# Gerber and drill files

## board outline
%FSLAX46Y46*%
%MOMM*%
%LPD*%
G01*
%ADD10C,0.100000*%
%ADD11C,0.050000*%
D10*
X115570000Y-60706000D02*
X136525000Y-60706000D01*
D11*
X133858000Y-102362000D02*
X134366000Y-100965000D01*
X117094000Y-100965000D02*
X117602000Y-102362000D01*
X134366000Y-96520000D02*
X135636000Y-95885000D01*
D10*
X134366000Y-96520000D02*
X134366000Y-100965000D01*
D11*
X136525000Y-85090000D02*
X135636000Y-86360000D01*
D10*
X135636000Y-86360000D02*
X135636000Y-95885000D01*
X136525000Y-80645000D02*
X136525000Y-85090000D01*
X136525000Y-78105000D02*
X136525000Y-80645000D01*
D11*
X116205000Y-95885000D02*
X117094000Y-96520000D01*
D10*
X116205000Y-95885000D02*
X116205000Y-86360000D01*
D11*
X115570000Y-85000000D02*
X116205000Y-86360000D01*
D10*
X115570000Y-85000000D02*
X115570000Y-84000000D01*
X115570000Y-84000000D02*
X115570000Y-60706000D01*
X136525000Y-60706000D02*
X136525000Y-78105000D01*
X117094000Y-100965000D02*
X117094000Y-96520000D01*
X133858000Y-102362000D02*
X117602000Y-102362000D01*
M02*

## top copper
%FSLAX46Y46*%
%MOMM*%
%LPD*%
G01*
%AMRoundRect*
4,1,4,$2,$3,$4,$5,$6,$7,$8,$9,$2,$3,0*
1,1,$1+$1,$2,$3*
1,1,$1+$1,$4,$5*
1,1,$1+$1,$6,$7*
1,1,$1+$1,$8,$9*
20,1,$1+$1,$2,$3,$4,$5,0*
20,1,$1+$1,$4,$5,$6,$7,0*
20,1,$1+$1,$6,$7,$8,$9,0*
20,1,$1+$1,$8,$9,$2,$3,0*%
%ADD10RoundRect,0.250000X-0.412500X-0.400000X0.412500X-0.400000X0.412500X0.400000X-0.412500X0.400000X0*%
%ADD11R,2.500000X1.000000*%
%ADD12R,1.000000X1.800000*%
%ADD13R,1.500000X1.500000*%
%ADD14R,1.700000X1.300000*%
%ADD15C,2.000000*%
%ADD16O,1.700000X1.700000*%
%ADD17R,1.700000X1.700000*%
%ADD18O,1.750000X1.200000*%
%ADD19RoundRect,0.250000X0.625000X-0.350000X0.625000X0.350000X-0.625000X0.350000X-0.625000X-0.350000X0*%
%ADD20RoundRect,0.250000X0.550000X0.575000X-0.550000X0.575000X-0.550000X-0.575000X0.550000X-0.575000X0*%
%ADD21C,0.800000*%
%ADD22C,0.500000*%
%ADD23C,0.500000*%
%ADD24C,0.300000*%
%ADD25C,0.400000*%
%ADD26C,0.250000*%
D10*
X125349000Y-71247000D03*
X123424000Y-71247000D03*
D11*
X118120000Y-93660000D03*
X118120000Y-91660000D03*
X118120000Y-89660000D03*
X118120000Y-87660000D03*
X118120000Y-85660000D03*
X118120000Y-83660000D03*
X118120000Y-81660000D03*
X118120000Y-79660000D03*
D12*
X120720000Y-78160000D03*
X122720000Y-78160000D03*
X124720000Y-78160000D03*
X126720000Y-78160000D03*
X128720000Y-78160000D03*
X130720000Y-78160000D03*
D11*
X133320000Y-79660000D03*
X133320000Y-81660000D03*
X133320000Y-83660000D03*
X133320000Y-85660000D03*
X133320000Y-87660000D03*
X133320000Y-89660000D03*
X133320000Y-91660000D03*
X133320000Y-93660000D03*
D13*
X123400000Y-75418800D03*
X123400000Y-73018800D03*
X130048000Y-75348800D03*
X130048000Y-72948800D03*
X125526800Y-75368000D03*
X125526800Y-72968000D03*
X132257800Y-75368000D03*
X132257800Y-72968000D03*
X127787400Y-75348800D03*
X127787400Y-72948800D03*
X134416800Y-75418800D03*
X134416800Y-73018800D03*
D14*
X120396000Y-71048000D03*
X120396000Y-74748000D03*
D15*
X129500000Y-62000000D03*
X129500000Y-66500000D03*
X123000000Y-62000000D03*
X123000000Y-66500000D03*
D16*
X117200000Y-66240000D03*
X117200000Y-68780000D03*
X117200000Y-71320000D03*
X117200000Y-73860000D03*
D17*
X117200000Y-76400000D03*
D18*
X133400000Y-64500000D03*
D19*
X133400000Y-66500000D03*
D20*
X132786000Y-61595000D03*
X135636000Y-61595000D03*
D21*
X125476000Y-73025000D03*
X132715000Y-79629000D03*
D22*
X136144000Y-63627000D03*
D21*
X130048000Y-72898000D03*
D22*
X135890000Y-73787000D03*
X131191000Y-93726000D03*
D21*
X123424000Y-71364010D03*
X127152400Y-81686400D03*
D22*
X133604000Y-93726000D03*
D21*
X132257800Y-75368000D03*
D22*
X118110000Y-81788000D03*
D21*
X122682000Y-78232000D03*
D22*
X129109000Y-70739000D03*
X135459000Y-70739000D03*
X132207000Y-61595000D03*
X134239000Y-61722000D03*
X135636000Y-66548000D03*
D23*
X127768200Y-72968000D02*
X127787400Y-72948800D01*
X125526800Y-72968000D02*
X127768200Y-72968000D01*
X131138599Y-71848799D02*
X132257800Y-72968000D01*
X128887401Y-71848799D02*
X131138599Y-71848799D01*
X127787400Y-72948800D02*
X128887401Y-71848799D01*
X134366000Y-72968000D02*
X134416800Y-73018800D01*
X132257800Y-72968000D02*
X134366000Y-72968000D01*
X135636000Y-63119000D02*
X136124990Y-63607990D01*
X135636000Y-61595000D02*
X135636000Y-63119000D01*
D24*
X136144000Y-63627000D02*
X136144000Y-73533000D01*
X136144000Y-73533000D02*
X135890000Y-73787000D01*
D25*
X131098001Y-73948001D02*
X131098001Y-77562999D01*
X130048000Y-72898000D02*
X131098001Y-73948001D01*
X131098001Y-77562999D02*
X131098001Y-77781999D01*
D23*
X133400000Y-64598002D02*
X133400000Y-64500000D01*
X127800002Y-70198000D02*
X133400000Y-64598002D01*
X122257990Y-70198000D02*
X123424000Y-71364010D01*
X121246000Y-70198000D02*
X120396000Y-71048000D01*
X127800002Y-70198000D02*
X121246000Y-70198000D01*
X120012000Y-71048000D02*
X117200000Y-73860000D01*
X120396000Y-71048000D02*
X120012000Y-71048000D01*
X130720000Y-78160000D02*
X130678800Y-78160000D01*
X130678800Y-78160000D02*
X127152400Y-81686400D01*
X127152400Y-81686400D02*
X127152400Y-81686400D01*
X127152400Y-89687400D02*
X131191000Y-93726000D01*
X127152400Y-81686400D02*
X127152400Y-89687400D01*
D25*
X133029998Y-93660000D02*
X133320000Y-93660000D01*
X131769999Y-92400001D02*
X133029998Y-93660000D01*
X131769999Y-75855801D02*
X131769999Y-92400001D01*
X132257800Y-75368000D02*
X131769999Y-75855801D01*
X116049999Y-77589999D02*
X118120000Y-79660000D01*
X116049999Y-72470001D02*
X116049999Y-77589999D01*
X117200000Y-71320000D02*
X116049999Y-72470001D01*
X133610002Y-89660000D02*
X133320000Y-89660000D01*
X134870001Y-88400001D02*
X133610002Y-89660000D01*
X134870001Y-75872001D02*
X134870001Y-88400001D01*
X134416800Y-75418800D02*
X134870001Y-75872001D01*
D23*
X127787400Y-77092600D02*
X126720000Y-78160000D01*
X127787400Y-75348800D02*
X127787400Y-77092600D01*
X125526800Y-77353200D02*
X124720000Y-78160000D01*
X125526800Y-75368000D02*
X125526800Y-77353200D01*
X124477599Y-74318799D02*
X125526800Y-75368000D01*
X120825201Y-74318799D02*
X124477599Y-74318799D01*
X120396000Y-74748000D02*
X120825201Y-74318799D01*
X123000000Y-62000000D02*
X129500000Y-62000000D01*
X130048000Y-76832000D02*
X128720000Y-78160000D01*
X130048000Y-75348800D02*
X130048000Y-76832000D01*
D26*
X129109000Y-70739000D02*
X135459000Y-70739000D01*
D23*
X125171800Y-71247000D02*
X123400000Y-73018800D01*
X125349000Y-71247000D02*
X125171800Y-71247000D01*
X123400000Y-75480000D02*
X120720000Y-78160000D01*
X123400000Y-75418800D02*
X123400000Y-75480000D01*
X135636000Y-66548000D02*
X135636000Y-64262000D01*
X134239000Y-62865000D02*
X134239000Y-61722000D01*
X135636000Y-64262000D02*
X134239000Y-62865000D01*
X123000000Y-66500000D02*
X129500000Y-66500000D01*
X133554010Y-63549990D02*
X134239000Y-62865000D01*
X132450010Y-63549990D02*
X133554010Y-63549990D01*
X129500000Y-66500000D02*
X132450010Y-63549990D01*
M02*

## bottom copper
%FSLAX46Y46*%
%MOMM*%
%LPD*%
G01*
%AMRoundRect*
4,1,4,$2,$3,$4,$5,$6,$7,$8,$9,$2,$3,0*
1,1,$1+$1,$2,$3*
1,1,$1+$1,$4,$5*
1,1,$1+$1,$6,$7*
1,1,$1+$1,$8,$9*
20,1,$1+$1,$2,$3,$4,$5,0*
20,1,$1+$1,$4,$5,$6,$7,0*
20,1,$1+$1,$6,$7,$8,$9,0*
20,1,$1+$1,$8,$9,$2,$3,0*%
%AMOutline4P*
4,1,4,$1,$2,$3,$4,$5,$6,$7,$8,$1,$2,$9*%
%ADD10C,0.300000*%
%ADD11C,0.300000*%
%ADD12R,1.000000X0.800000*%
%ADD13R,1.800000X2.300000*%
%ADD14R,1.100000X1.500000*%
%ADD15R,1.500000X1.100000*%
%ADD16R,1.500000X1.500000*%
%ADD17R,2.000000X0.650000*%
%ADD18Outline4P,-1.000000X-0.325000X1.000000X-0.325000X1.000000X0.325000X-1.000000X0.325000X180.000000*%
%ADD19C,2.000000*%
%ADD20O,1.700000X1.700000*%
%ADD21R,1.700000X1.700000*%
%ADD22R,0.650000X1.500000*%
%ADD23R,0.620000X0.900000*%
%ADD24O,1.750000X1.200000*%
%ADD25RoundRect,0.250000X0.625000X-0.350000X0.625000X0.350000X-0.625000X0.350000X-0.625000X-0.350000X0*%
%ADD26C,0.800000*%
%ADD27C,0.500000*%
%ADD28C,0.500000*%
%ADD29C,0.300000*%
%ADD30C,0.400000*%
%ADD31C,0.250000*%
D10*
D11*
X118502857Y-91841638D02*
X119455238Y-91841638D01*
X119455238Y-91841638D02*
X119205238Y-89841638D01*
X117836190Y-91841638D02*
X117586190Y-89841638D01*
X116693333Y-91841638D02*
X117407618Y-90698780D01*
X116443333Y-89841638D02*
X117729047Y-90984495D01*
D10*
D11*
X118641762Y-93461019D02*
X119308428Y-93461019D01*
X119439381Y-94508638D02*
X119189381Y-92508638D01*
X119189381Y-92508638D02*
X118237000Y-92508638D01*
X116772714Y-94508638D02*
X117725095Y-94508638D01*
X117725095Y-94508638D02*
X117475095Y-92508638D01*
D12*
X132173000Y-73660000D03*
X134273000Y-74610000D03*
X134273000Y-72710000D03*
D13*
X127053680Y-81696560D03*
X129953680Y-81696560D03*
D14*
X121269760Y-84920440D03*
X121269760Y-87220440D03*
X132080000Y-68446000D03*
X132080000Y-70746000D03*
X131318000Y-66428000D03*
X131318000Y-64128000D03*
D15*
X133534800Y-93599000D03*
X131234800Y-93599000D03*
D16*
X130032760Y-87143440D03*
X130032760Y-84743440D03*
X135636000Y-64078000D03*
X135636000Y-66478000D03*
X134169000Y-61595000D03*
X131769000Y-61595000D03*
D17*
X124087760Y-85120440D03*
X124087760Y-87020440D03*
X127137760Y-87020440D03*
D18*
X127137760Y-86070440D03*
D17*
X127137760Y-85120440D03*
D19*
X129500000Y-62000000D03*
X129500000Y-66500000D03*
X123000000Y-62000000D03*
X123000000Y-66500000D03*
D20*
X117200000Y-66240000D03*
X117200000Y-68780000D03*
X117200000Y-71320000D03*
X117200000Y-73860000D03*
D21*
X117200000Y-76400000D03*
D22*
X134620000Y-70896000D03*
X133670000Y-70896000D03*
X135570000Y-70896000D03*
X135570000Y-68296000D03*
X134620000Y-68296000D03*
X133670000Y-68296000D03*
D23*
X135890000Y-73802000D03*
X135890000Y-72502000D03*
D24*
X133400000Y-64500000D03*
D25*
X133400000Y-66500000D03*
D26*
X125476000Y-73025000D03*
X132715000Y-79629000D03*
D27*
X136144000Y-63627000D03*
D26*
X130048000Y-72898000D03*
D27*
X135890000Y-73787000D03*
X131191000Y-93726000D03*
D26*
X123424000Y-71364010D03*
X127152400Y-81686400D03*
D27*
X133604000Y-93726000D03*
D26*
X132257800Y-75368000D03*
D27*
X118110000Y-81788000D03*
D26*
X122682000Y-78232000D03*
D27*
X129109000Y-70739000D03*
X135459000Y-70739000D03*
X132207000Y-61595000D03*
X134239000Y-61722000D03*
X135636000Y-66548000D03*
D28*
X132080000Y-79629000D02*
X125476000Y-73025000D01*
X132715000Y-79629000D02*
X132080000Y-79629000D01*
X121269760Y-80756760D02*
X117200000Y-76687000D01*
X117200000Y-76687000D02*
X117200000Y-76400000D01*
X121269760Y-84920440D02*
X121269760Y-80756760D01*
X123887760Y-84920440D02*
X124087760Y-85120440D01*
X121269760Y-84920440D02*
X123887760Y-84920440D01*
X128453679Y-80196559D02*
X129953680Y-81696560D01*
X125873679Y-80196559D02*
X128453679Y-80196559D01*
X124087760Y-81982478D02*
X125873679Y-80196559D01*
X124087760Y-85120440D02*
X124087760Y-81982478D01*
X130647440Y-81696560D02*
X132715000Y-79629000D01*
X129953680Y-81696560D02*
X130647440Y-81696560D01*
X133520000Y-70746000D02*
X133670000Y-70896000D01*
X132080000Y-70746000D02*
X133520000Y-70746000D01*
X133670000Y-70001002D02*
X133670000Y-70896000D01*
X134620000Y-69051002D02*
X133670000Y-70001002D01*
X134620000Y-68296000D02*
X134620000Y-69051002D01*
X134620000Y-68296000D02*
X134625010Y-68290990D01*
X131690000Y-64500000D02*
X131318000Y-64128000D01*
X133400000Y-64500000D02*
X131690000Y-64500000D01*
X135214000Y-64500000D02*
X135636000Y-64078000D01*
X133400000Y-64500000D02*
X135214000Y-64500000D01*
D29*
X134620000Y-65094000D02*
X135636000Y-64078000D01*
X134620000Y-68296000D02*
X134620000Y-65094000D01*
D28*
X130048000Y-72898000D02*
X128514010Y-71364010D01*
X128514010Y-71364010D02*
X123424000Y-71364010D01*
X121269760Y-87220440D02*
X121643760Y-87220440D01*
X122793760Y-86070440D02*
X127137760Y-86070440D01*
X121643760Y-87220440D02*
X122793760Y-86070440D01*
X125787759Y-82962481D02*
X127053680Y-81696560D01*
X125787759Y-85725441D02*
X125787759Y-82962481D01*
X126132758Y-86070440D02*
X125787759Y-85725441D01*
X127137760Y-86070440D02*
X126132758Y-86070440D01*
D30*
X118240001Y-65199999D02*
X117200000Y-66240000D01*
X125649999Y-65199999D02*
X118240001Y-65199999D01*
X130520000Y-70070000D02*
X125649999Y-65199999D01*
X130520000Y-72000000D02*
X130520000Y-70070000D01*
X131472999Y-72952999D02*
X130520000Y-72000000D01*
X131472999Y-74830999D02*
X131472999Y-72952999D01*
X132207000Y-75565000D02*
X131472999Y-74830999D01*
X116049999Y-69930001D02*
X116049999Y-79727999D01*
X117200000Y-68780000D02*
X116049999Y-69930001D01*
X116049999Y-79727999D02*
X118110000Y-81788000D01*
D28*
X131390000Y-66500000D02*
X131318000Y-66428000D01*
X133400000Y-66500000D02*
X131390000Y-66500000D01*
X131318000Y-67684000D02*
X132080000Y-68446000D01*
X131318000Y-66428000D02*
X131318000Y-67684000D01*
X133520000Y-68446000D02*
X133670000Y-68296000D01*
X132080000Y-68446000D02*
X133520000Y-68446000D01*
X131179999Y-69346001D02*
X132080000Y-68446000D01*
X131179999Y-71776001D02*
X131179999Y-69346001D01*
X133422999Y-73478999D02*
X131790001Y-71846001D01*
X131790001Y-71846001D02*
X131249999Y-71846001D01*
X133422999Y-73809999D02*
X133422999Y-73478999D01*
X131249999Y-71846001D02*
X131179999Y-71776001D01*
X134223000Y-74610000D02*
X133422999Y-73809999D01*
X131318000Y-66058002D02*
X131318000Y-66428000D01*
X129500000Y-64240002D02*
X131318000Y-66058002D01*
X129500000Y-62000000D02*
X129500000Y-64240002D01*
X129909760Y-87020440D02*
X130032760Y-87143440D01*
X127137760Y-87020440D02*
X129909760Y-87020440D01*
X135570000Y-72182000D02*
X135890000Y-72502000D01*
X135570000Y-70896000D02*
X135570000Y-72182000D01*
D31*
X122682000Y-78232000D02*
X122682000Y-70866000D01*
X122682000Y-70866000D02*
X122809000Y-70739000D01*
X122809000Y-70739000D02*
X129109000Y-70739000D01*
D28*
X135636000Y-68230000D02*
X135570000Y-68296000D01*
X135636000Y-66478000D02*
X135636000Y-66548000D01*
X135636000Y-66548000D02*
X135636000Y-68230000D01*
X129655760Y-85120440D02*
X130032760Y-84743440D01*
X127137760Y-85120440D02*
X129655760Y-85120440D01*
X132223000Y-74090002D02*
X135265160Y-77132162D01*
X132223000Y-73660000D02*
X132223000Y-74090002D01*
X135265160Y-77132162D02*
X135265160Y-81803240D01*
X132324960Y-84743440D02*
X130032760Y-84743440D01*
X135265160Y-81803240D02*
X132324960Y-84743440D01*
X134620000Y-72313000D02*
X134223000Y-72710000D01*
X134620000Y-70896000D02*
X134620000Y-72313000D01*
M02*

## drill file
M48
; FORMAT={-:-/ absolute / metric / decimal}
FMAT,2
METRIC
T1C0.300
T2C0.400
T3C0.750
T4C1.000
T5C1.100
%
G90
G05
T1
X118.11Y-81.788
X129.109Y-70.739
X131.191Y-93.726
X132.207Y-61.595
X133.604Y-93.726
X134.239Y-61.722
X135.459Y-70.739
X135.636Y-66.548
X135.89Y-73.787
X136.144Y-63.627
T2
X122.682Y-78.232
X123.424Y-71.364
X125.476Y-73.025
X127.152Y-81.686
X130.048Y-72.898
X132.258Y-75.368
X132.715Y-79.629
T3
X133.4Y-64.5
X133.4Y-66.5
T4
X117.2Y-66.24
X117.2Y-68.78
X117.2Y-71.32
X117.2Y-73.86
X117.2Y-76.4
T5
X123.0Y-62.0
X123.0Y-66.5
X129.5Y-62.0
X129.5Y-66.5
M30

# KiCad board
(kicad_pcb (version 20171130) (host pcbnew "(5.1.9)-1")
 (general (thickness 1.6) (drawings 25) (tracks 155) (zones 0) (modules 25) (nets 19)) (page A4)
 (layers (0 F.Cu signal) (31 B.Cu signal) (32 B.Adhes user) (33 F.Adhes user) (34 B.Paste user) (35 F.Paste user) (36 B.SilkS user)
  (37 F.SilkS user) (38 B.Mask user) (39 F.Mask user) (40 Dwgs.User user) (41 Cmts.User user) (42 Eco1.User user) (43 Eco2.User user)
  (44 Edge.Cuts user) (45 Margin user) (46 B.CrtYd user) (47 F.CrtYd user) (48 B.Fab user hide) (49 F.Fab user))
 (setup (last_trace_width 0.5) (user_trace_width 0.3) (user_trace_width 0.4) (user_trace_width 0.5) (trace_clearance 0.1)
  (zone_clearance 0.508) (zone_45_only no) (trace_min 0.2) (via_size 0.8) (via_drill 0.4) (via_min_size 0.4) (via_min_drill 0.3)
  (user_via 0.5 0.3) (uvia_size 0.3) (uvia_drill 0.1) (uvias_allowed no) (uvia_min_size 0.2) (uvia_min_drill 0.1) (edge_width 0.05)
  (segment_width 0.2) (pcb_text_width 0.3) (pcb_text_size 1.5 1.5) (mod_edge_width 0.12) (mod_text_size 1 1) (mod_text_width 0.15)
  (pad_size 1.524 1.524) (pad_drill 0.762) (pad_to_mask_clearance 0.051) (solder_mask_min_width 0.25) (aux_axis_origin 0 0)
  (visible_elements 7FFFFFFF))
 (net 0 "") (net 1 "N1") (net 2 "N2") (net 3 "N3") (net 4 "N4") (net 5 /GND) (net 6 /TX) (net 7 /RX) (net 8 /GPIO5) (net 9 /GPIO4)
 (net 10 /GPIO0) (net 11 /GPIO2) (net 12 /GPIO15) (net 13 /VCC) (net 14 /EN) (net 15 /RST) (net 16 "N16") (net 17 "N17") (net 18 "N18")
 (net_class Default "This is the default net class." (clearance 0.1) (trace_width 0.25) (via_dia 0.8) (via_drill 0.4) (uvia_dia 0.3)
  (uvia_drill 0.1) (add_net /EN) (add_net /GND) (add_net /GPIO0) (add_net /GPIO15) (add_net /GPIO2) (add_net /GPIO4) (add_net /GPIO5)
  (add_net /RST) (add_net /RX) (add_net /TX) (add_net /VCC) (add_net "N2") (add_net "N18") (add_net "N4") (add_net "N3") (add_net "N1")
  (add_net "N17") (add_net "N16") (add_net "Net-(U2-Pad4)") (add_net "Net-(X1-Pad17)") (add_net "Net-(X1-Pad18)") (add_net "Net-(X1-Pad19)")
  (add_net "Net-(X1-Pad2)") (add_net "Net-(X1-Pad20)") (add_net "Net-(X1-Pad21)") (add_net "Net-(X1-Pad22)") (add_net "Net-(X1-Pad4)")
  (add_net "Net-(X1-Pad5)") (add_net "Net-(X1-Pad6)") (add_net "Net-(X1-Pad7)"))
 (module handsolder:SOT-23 (layer B.Cu) (at 133.223 73.66 180)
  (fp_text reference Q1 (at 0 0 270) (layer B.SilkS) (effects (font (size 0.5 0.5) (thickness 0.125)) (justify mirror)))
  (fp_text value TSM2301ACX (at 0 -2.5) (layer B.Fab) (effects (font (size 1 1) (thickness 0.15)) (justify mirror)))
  (pad 3 smd rect (at 1.05 0 180) (size 1 0.8) (layers B.Cu B.Paste B.Mask) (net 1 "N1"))
  (pad 2 smd rect (at -1.05 -0.95 180) (size 1 0.8) (layers B.Cu B.Paste B.Mask) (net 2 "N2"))
  (pad 1 smd rect (at -1.05 0.95 180) (size 1 0.8) (layers B.Cu B.Paste B.Mask) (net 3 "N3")))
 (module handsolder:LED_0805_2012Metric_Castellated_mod (layer F.Cu) (at 124.3865 71.247)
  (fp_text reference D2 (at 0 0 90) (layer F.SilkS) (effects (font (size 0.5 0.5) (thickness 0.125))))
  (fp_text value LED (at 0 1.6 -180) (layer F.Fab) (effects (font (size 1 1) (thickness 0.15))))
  (pad 2 smd roundrect (at 0.9625 0) (size 1.325 1.3) (layers F.Cu F.Paste F.Mask) (roundrect_rratio 0.1923076923076923) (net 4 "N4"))
  (pad 1 smd roundrect (at -0.9625 0) (size 1.325 1.3) (layers F.Cu F.Paste F.Mask) (roundrect_rratio 0.1923076923076923) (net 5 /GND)))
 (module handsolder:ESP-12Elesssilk (layer F.Cu) (at 125.72 90.16 180)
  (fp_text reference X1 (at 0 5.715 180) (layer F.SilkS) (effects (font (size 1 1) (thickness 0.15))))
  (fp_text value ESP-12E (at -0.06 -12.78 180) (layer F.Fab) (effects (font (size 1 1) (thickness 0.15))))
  (pad 22 smd rect (at 7.6 -3.5 180) (size 2.5 1) (layers F.Cu F.Paste F.Mask))
  (pad 21 smd rect (at 7.6 -1.5 180) (size 2.5 1) (layers F.Cu F.Paste F.Mask))
  (pad 20 smd rect (at 7.6 0.5 180) (size 2.5 1) (layers F.Cu F.Paste F.Mask))
  (pad 19 smd rect (at 7.6 2.5 180) (size 2.5 1) (layers F.Cu F.Paste F.Mask))
  (pad 18 smd rect (at 7.6 4.5 180) (size 2.5 1) (layers F.Cu F.Paste F.Mask))
  (pad 17 smd rect (at 7.6 6.5 180) (size 2.5 1) (layers F.Cu F.Paste F.Mask))
  (pad 16 smd rect (at 7.6 8.5 180) (size 2.5 1) (layers F.Cu F.Paste F.Mask) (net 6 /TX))
  (pad 15 smd rect (at 7.6 10.5 180) (size 2.5 1) (layers F.Cu F.Paste F.Mask) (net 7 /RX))
  (pad 14 smd rect (at 5 12 180) (size 1 1.8) (layers F.Cu F.Paste F.Mask) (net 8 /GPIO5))
  (pad 13 smd rect (at 3 12 180) (size 1 1.8) (layers F.Cu F.Paste F.Mask) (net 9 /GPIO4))
  (pad 12 smd rect (at 1 12 180) (size 1 1.8) (layers F.Cu F.Paste F.Mask) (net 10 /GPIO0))
  (pad 11 smd rect (at -1 12 180) (size 1 1.8) (layers F.Cu F.Paste F.Mask) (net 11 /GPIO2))
  (pad 10 smd rect (at -3 12 180) (size 1 1.8) (layers F.Cu F.Paste F.Mask) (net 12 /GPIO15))
  (pad 9 smd rect (at -5 12 180) (size 1 1.8) (layers F.Cu F.Paste F.Mask) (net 5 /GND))
  (pad 8 smd rect (at -7.6 10.5 180) (size 2.5 1) (layers F.Cu F.Paste F.Mask) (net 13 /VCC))
  (pad 7 smd rect (at -7.6 8.5 180) (size 2.5 1) (layers F.Cu F.Paste F.Mask))
  (pad 6 smd rect (at -7.6 6.5 180) (size 2.5 1) (layers F.Cu F.Paste F.Mask))
  (pad 5 smd rect (at -7.6 4.5 180) (size 2.5 1) (layers F.Cu F.Paste F.Mask))
  (pad 4 smd rect (at -7.6 2.5 180) (size 2.5 1) (layers F.Cu F.Paste F.Mask))
  (pad 3 smd rect (at -7.6 0.5 180) (size 2.5 1) (layers F.Cu F.Paste F.Mask) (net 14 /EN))
  (pad 2 smd rect (at -7.6 -1.5 180) (size 2.5 1) (layers F.Cu F.Paste F.Mask))
  (pad 1 smd rect (at -7.6 -3.5 180) (size 2.5 1) (layers F.Cu F.Paste F.Mask) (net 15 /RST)))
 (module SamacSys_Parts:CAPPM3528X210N (layer B.Cu) (at 128.50368 81.69656 180)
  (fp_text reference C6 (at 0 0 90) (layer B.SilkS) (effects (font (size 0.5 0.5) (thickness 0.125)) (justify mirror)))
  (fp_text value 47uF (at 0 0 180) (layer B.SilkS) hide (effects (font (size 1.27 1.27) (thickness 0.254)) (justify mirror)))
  (pad 2 smd rect (at 1.45 0 180) (size 1.8 2.3) (layers B.Cu B.Paste B.Mask) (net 5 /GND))
  (pad 1 smd rect (at -1.45 0 180) (size 1.8 2.3) (layers B.Cu B.Paste B.Mask) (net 13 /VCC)))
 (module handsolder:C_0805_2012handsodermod (layer B.Cu) (at 121.26976 86.07044 90)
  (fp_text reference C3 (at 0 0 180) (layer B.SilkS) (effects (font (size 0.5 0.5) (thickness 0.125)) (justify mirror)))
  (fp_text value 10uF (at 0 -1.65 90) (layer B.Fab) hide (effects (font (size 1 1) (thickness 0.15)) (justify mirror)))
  (pad 2 smd rect (at 1.15 0 90) (size 1.5 1.1) (layers B.Cu B.Paste B.Mask) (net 13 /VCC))
  (pad 1 smd rect (at -1.15 0 90) (size 1.5 1.1) (layers B.Cu B.Paste B.Mask) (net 5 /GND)))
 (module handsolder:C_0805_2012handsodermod (layer B.Cu) (at 132.08 69.596 90)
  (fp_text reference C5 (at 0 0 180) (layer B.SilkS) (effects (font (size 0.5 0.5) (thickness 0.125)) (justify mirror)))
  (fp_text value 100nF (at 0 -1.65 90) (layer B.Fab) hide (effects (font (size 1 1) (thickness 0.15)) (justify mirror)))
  (pad 2 smd rect (at 1.15 0 90) (size 1.5 1.1) (layers B.Cu B.Paste B.Mask) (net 2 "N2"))
  (pad 1 smd rect (at -1.15 0 90) (size 1.5 1.1) (layers B.Cu B.Paste B.Mask) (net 5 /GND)))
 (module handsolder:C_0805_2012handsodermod (layer B.Cu) (at 131.318 65.278 270)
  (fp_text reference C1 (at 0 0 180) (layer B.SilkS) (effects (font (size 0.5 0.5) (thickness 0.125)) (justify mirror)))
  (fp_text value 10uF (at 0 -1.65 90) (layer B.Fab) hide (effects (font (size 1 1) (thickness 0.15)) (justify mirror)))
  (pad 2 smd rect (at 1.15 0 270) (size 1.5 1.1) (layers B.Cu B.Paste B.Mask) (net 2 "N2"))
  (pad 1 smd rect (at -1.15 0 270) (size 1.5 1.1) (layers B.Cu B.Paste B.Mask) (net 5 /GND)))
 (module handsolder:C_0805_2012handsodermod (layer B.Cu) (at 132.3848 93.599)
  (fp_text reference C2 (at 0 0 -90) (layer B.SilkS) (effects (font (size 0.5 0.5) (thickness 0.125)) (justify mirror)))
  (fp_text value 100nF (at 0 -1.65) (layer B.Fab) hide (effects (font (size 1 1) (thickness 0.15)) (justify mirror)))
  (pad 2 smd rect (at 1.15 0) (size 1.5 1.1) (layers B.Cu B.Paste B.Mask) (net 15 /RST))
  (pad 1 smd rect (at -1.15 0) (size 1.5 1.1) (layers B.Cu B.Paste B.Mask) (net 5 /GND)))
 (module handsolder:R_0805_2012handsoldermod (layer F.Cu) (at 123.4 74.2188 270)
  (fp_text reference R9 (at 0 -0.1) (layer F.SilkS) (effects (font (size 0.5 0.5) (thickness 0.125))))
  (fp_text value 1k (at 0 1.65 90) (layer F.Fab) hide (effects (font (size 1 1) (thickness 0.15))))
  (pad 2 smd rect (at 1.2 0 270) (size 1.5 1.5) (layers F.Cu F.Paste F.Mask) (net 8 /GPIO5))
  (pad 1 smd rect (at -1.2 0 270) (size 1.5 1.5) (layers F.Cu F.Paste F.Mask) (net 4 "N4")))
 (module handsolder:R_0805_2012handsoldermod (layer B.Cu) (at 130.03276 85.94344 270)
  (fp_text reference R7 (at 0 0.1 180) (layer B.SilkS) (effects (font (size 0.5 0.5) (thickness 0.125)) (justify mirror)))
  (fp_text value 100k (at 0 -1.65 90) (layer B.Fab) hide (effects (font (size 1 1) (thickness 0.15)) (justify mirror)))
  (pad 2 smd rect (at 1.2 0 270) (size 1.5 1.5) (layers B.Cu B.Paste B.Mask) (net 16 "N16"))
  (pad 1 smd rect (at -1.2 0 270) (size 1.5 1.5) (layers B.Cu B.Paste B.Mask) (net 1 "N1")))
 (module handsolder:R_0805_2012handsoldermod (layer B.Cu) (at 135.636 65.278 90)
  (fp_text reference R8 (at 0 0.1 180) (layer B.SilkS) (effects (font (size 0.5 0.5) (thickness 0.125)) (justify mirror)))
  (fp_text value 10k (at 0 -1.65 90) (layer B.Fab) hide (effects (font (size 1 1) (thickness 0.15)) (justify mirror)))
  (pad 2 smd rect (at 1.2 0 90) (size 1.5 1.5) (layers B.Cu B.Paste B.Mask) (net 5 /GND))
  (pad 1 smd rect (at -1.2 0 90) (size 1.5 1.5) (layers B.Cu B.Paste B.Mask) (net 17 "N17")))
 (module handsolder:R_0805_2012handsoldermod (layer B.Cu) (at 132.969 61.595)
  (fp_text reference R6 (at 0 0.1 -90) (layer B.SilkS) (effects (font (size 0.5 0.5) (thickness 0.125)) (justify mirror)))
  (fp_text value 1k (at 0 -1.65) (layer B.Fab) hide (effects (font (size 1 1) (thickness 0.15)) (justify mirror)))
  (pad 2 smd rect (at 1.2 0) (size 1.5 1.5) (layers B.Cu B.Paste B.Mask) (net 17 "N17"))
  (pad 1 smd rect (at -1.2 0) (size 1.5 1.5) (layers B.Cu B.Paste B.Mask) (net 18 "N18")))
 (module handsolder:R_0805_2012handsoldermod (layer F.Cu) (at 130.048 74.1488 270)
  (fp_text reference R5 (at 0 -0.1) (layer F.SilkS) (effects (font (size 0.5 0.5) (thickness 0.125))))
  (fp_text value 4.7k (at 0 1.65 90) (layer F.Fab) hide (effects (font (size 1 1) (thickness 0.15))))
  (pad 2 smd rect (at 1.2 0 270) (size 1.5 1.5) (layers F.Cu F.Paste F.Mask) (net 12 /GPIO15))
  (pad 1 smd rect (at -1.2 0 270) (size 1.5 1.5) (layers F.Cu F.Paste F.Mask) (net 5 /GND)))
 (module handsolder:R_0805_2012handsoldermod (layer F.Cu) (at 125.5268 74.168 270)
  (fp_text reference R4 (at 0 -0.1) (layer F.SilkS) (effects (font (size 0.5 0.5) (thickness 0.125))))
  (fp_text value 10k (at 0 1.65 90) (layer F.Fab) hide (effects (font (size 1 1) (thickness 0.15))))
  (pad 2 smd rect (at 1.2 0 270) (size 1.5 1.5) (layers F.Cu F.Paste F.Mask) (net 10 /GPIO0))
  (pad 1 smd rect (at -1.2 0 270) (size 1.5 1.5) (layers F.Cu F.Paste F.Mask) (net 13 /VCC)))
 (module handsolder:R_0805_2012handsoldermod (layer F.Cu) (at 132.2578 74.168 270)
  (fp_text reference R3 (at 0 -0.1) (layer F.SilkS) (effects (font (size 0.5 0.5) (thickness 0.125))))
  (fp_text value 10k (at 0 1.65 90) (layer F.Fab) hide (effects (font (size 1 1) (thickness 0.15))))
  (pad 2 smd rect (at 1.2 0 270) (size 1.5 1.5) (layers F.Cu F.Paste F.Mask) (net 15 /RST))
  (pad 1 smd rect (at -1.2 0 270) (size 1.5 1.5) (layers F.Cu F.Paste F.Mask) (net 13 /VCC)))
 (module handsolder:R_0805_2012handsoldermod (layer F.Cu) (at 127.7874 74.1488 270)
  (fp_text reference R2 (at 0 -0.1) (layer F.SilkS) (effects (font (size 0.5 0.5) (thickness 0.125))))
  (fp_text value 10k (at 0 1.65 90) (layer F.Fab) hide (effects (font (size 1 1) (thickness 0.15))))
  (pad 2 smd rect (at 1.2 0 270) (size 1.5 1.5) (layers F.Cu F.Paste F.Mask) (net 11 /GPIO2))
  (pad 1 smd rect (at -1.2 0 270) (size 1.5 1.5) (layers F.Cu F.Paste F.Mask) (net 13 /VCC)))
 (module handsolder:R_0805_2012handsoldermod (layer F.Cu) (at 134.4168 74.2188 270)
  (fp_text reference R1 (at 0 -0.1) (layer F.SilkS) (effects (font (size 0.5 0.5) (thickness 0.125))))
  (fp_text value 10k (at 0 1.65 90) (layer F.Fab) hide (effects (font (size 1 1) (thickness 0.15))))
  (pad 2 smd rect (at 1.2 0 270) (size 1.5 1.5) (layers F.Cu F.Paste F.Mask) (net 14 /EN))
  (pad 1 smd rect (at -1.2 0 270) (size 1.5 1.5) (layers F.Cu F.Paste F.Mask) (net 13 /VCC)))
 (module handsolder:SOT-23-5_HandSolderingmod (layer B.Cu) (at 125.58776 86.07044 180)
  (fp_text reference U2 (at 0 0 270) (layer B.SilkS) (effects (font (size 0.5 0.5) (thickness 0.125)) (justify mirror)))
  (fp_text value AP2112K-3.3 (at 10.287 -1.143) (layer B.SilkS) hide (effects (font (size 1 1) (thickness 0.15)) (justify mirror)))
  (pad 5 smd rect (at 1.5 0.95 180) (size 2 0.65) (layers B.Cu B.Paste B.Mask) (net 13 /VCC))
  (pad 4 smd rect (at 1.5 -0.95 180) (size 2 0.65) (layers B.Cu B.Paste B.Mask))
  (pad 3 smd rect (at -1.55 -0.95 180) (size 2 0.65) (layers B.Cu B.Paste B.Mask) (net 16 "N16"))
  (pad 2 smd trapezoid (at -1.55 0 180) (size 2 0.65) (layers B.Cu B.Paste B.Mask) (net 5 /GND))
  (pad 1 smd rect (at -1.55 0.95 180) (size 2 0.65) (layers B.Cu B.Paste B.Mask) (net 1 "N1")))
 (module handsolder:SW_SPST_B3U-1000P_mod (layer F.Cu) (at 120.396 72.898 90)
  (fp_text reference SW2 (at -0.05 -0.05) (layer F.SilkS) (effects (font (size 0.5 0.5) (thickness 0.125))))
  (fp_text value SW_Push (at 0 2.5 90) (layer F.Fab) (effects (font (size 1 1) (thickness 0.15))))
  (pad 2 smd rect (at 1.85 0 90) (size 1.3 1.7) (layers F.Cu F.Paste F.Mask) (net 5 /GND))
  (pad 1 smd rect (at -1.85 0 90) (size 1.3 1.7) (layers F.Cu F.Paste F.Mask) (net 10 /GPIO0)))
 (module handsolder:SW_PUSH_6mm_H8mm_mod (layer F.Cu) (at 123 62)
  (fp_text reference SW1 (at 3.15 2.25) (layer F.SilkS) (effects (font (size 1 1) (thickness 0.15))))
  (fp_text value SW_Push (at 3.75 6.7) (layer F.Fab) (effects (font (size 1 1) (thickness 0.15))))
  (pad 1 thru_hole circle (at 6.5 0 90) (size 2 2) (drill 1.1) (layers *.Cu *.Mask) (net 2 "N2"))
  (pad 2 thru_hole circle (at 6.5 4.5 90) (size 2 2) (drill 1.1) (layers *.Cu *.Mask) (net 17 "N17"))
  (pad 1 thru_hole circle (at 0 0 90) (size 2 2) (drill 1.1) (layers *.Cu *.Mask) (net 2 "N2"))
  (pad 2 thru_hole circle (at 0 4.5 90) (size 2 2) (drill 1.1) (layers *.Cu *.Mask) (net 17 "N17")))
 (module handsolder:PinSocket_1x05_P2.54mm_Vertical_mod (layer F.Cu) (at 117.2 76.4 180)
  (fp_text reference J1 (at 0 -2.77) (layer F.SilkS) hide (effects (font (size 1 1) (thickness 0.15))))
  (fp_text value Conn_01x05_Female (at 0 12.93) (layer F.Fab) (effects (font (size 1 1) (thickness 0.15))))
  (pad 5 thru_hole oval (at 0 10.16 180) (size 1.7 1.7) (drill 1) (layers *.Cu *.Mask) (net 15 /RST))
  (pad 4 thru_hole oval (at 0 7.62 180) (size 1.7 1.7) (drill 1) (layers *.Cu *.Mask) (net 6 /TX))
  (pad 3 thru_hole oval (at 0 5.08 180) (size 1.7 1.7) (drill 1) (layers *.Cu *.Mask) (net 7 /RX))
  (pad 2 thru_hole oval (at 0 2.54 180) (size 1.7 1.7) (drill 1) (layers *.Cu *.Mask) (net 5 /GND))
  (pad 1 thru_hole rect (at 0 0 180) (size 1.7 1.7) (drill 1) (layers *.Cu *.Mask) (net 13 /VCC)))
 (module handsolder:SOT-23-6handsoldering (layer B.Cu) (at 134.62 69.596 270)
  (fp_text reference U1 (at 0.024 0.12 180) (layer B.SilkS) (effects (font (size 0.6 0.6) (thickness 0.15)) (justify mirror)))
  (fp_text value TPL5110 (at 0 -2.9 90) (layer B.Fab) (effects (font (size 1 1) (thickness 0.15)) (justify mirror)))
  (pad 5 smd rect (at 1.3 0 270) (size 1.5 0.65) (layers B.Cu B.Paste B.Mask) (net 3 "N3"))
  (pad 6 smd rect (at 1.3 0.95 270) (size 1.5 0.65) (layers B.Cu B.Paste B.Mask) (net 5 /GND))
  (pad 4 smd rect (at 1.3 -0.95 270) (size 1.5 0.65) (layers B.Cu B.Paste B.Mask) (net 9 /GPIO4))
  (pad 3 smd rect (at -1.3 -0.95 270) (size 1.5 0.65) (layers B.Cu B.Paste B.Mask) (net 17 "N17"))
  (pad 2 smd rect (at -1.3 0 270) (size 1.5 0.65) (layers B.Cu B.Paste B.Mask) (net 5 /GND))
  (pad 1 smd rect (at -1.3 0.95 270) (size 1.5 0.65) (layers B.Cu B.Paste B.Mask) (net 2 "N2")))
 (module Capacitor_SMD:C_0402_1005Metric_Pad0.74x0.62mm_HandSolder (layer B.Cu) (at 135.89 73.152 270)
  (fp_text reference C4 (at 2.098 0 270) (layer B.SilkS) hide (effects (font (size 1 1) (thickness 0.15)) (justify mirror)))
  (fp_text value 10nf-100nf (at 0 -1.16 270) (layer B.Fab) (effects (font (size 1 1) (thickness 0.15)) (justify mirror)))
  (pad 2 smd rect (at 0.65 0 270) (size 0.9 0.62) (layers B.Cu B.Paste B.Mask) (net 5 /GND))
  (pad 1 smd rect (at -0.65 0 270) (size 0.9 0.62) (layers B.Cu B.Paste B.Mask) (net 9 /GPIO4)))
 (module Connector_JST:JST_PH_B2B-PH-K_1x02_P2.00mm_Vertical (layer F.Cu) (at 133.4 66.5 90)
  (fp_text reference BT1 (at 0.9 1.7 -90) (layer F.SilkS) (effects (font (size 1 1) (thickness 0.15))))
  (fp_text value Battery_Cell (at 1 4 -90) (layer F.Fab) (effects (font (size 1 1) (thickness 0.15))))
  (pad 2 thru_hole oval (at 2 0 90) (size 1.2 1.75) (drill 0.75) (layers *.Cu *.Mask) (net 5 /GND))
  (pad 1 thru_hole roundrect (at 0 0 90) (size 1.2 1.75) (drill 0.75) (layers *.Cu *.Mask) (roundrect_rratio 0.208333) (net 2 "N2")))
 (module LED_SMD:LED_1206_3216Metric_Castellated (layer F.Cu) (at 134.211 61.595 180)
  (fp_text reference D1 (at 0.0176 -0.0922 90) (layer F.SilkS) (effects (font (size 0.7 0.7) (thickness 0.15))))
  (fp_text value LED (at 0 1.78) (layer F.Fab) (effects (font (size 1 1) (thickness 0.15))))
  (pad 2 smd roundrect (at 1.425 0 180) (size 1.6 1.65) (layers F.Cu F.Paste F.Mask) (roundrect_rratio 0.15625) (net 18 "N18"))
  (pad 1 smd roundrect (at -1.425 0 180) (size 1.6 1.65) (layers F.Cu F.Paste F.Mask) (roundrect_rratio 0.15625) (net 5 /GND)))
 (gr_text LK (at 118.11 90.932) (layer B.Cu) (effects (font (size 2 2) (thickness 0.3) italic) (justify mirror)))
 (gr_line (start 115.57 60.706) (end 136.525 60.706) (layer Edge.Cuts) (width 0.1))
 (gr_line (start 133.858 102.362) (end 134.366 100.965) (layer Edge.Cuts) (width 0.05))
 (gr_line (start 117.094 100.965) (end 117.602 102.362) (layer Edge.Cuts) (width 0.05))
 (gr_line (start 134.366 96.52) (end 135.636 95.885) (layer Edge.Cuts) (width 0.05))
 (gr_line (start 134.366 96.52) (end 134.366 100.965) (layer Edge.Cuts) (width 0.1))
 (gr_line (start 136.525 85.09) (end 135.636 86.36) (layer Edge.Cuts) (width 0.05))
 (gr_line (start 135.636 86.36) (end 135.636 95.885) (layer Edge.Cuts) (width 0.1))
 (gr_line (start 136.525 80.645) (end 136.525 85.09) (layer Edge.Cuts) (width 0.1))
 (gr_line (start 136.525 78.105) (end 136.525 80.645) (layer Edge.Cuts) (width 0.1))
 (gr_line (start 116.205 95.885) (end 117.094 96.52) (layer Edge.Cuts) (width 0.05))
 (gr_line (start 116.205 95.885) (end 116.205 86.36) (layer Edge.Cuts) (width 0.1))
 (gr_line (start 115.57 85) (end 116.205 86.36) (layer Edge.Cuts) (width 0.05))
 (gr_line (start 115.57 85) (end 115.57 84) (layer Edge.Cuts) (width 0.1))
 (gr_line (start 115.57 84) (end 115.57 60.706) (layer Edge.Cuts) (width 0.1))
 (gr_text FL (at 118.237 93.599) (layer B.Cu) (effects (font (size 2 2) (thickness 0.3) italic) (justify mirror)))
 (gr_line (start 136.525 60.706) (end 136.525 78.105) (layer Edge.Cuts) (width 0.1))
 (gr_line (start 117.094 100.965) (end 117.094 96.52) (layer Edge.Cuts) (width 0.1))
 (gr_line (start 133.858 102.362) (end 117.602 102.362) (layer Edge.Cuts) (width 0.1))
 (via (at 125.476 73.025) (size 0.8) (drill 0.4) (layers F.Cu B.Cu) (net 13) (status 30))
 (via (at 132.715 79.629) (size 0.8) (drill 0.4) (layers F.Cu B.Cu) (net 13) (status 30))
 (segment (start 132.08 79.629) (end 125.476 73.025) (width 0.5) (layer B.Cu) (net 13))
 (segment (start 132.715 79.629) (end 132.08 79.629) (width 0.5) (layer B.Cu) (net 13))
 (segment (start 127.7682 72.968) (end 127.7874 72.9488) (width 0.5) (layer F.Cu) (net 13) (status 30))
 (segment (start 125.5268 72.968) (end 127.7682 72.968) (width 0.5) (layer F.Cu) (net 13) (status 30))
 (segment (start 131.138599 71.848799) (end 132.2578 72.968) (width 0.5) (layer F.Cu) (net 13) (status 20))
 (segment (start 128.887401 71.848799) (end 131.138599 71.848799) (width 0.5) (layer F.Cu) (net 13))
 (segment (start 127.7874 72.9488) (end 128.887401 71.848799) (width 0.5) (layer F.Cu) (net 13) (status 10))
 (segment (start 134.366 72.968) (end 134.4168 73.0188) (width 0.5) (layer F.Cu) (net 13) (status 30))
 (segment (start 132.2578 72.968) (end 134.366 72.968) (width 0.5) (layer F.Cu) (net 13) (status 30))
 (segment (start 121.26976 80.75676) (end 117.2 76.687) (width 0.5) (layer B.Cu) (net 13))
 (segment (start 117.2 76.687) (end 117.2 76.4) (width 0.5) (layer B.Cu) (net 13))
 (segment (start 121.26976 84.92044) (end 121.26976 80.75676) (width 0.5) (layer B.Cu) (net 13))
 (segment (start 123.88776 84.92044) (end 124.08776 85.12044) (width 0.5) (layer B.Cu) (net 13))
 (segment (start 121.26976 84.92044) (end 123.88776 84.92044) (width 0.5) (layer B.Cu) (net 13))
 (segment (start 128.453679 80.196559) (end 129.95368 81.69656) (width 0.5) (layer B.Cu) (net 13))
 (segment (start 125.873679 80.196559) (end 128.453679 80.196559) (width 0.5) (layer B.Cu) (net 13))
 (segment (start 124.08776 81.982478) (end 125.873679 80.196559) (width 0.5) (layer B.Cu) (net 13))
 (segment (start 124.08776 85.12044) (end 124.08776 81.982478) (width 0.5) (layer B.Cu) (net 13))
 (segment (start 130.64744 81.69656) (end 132.715 79.629) (width 0.5) (layer B.Cu) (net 13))
 (segment (start 129.95368 81.69656) (end 130.64744 81.69656) (width 0.5) (layer B.Cu) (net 13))
 (via (at 136.144 63.627) (size 0.5) (drill 0.3) (layers F.Cu B.Cu) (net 5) (status 30))
 (segment (start 133.52 70.746) (end 133.67 70.896) (width 0.5) (layer B.Cu) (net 5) (status 30))
 (segment (start 132.08 70.746) (end 133.52 70.746) (width 0.5) (layer B.Cu) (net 5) (status 30))
 (segment (start 133.67 70.001002) (end 133.67 70.896) (width 0.5) (layer B.Cu) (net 5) (status 20))
 (segment (start 134.62 69.051002) (end 133.67 70.001002) (width 0.5) (layer B.Cu) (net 5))
 (segment (start 134.62 68.296) (end 134.62 69.051002) (width 0.5) (layer B.Cu) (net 5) (status 10))
 (segment (start 134.62 68.296) (end 134.62501 68.29099) (width 0.5) (layer B.Cu) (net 5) (status 30))
 (segment (start 131.69 64.5) (end 131.318 64.128) (width 0.5) (layer B.Cu) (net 5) (status 30))
 (segment (start 133.4 64.5) (end 131.69 64.5) (width 0.5) (layer B.Cu) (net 5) (status 30))
 (segment (start 135.214 64.5) (end 135.636 64.078) (width 0.5) (layer B.Cu) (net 5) (status 30))
 (segment (start 133.4 64.5) (end 135.214 64.5) (width 0.5) (layer B.Cu) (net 5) (status 30))
 (segment (start 134.62 65.094) (end 135.636 64.078) (width 0.3) (layer B.Cu) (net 5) (status 20))
 (segment (start 134.62 68.296) (end 134.62 65.094) (width 0.3) (layer B.Cu) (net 5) (status 10))
 (segment (start 135.636 63.119) (end 136.12499 63.60799) (width 0.5) (layer F.Cu) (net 5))
 (segment (start 135.636 61.595) (end 135.636 63.119) (width 0.5) (layer F.Cu) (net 5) (status 10))
 (via (at 130.048 72.898) (size 0.8) (drill 0.4) (layers F.Cu B.Cu) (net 5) (status 30))
 (segment (start 136.144 63.627) (end 136.144 73.533) (width 0.3) (layer F.Cu) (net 5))
 (segment (start 136.144 73.533) (end 135.89 73.787) (width 0.3) (layer F.Cu) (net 5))
 (via (at 135.89 73.787) (size 0.5) (drill 0.3) (layers F.Cu B.Cu) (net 5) (status 30))
 (segment (start 131.098001 73.948001) (end 131.098001 77.562999) (width 0.4) (layer F.Cu) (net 5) (status 20))
 (segment (start 130.048 72.898) (end 131.098001 73.948001) (width 0.4) (layer F.Cu) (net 5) (status 10))
 (segment (start 131.098001 77.562999) (end 131.098001 77.781999) (width 0.4) (layer F.Cu) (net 5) (status 30))
 (segment (start 133.4 64.598002) (end 133.4 64.5) (width 0.5) (layer F.Cu) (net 5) (status 30))
 (segment (start 127.800002 70.198) (end 133.4 64.598002) (width 0.5) (layer F.Cu) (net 5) (status 20))
 (via (at 131.191 93.726) (size 0.5) (drill 0.3) (layers F.Cu B.Cu) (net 5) (status 30))
 (via (at 123.424 71.36401) (size 0.8) (drill 0.4) (layers F.Cu B.Cu) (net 5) (status 30))
 (segment (start 122.25799 70.198) (end 123.424 71.36401) (width 0.5) (layer F.Cu) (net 5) (status 20))
 (segment (start 130.048 72.898) (end 128.51401 71.36401) (width 0.5) (layer B.Cu) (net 5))
 (segment (start 128.51401 71.36401) (end 123.424 71.36401) (width 0.5) (layer B.Cu) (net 5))
 (segment (start 121.246 70.198) (end 120.396 71.048) (width 0.5) (layer F.Cu) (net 5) (status 20))
 (segment (start 127.800002 70.198) (end 121.246 70.198) (width 0.5) (layer F.Cu) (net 5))
 (segment (start 120.012 71.048) (end 117.2 73.86) (width 0.5) (layer F.Cu) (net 5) (status 30))
 (segment (start 120.396 71.048) (end 120.012 71.048) (width 0.5) (layer F.Cu) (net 5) (status 30))
 (segment (start 121.26976 87.22044) (end 121.64376 87.22044) (width 0.5) (layer B.Cu) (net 5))
 (segment (start 122.79376 86.07044) (end 127.13776 86.07044) (width 0.5) (layer B.Cu) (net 5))
 (segment (start 121.64376 87.22044) (end 122.79376 86.07044) (width 0.5) (layer B.Cu) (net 5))
 (segment (start 125.787759 82.962481) (end 127.05368 81.69656) (width 0.5) (layer B.Cu) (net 5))
 (segment (start 125.787759 85.725441) (end 125.787759 82.962481) (width 0.5) (layer B.Cu) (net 5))
 (segment (start 126.132758 86.07044) (end 125.787759 85.725441) (width 0.5) (layer B.Cu) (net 5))
 (segment (start 127.13776 86.07044) (end 126.132758 86.07044) (width 0.5) (layer B.Cu) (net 5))
 (segment (start 130.72 78.16) (end 130.6788 78.16) (width 0.5) (layer F.Cu) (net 5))
 (segment (start 130.6788 78.16) (end 127.1524 81.6864) (width 0.5) (layer F.Cu) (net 5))
 (segment (start 127.1524 81.6864) (end 127.1524 81.6864) (width 0.5) (layer F.Cu) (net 5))
 (via (at 127.1524 81.6864) (size 0.8) (drill 0.4) (layers F.Cu B.Cu) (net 5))
 (segment (start 127.1524 89.6874) (end 131.191 93.726) (width 0.5) (layer F.Cu) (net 5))
 (segment (start 127.1524 81.6864) (end 127.1524 89.6874) (width 0.5) (layer F.Cu) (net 5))
 (via (at 133.604 93.726) (size 0.5) (drill 0.3) (layers F.Cu B.Cu) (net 15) (status 30))
 (segment (start 133.029998 93.66) (end 133.32 93.66) (width 0.4) (layer F.Cu) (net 15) (status 30))
 (segment (start 131.769999 92.400001) (end 133.029998 93.66) (width 0.4) (layer F.Cu) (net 15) (status 20))
 (segment (start 131.769999 75.855801) (end 131.769999 92.400001) (width 0.4) (layer F.Cu) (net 15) (status 10))
 (segment (start 132.2578 75.368) (end 131.769999 75.855801) (width 0.4) (layer F.Cu) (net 15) (status 30))
 (via (at 132.2578 75.368) (size 0.8) (drill 0.4) (layers F.Cu B.Cu) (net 15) (status 30))
 (segment (start 118.240001 65.199999) (end 117.2 66.24) (width 0.4) (layer B.Cu) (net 15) (status 20))
 (segment (start 125.649999 65.199999) (end 118.240001 65.199999) (width 0.4) (layer B.Cu) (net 15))
 (segment (start 130.52 70.07) (end 125.649999 65.199999) (width 0.4) (layer B.Cu) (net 15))
 (segment (start 130.52 72) (end 130.52 70.07) (width 0.4) (layer B.Cu) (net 15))
 (segment (start 131.472999 72.952999) (end 130.52 72) (width 0.4) (layer B.Cu) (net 15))
 (segment (start 131.472999 74.830999) (end 131.472999 72.952999) (width 0.4) (layer B.Cu) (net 15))
 (segment (start 132.207 75.565) (end 131.472999 74.830999) (width 0.4) (layer B.Cu) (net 15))
 (segment (start 116.049999 77.589999) (end 118.12 79.66) (width 0.4) (layer F.Cu) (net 7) (status 20))
 (segment (start 116.049999 72.470001) (end 116.049999 77.589999) (width 0.4) (layer F.Cu) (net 7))
 (segment (start 117.2 71.32) (end 116.049999 72.470001) (width 0.4) (layer F.Cu) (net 7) (status 10))
 (segment (start 116.049999 69.930001) (end 116.049999 79.727999) (width 0.4) (layer B.Cu) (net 6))
 (segment (start 117.2 68.78) (end 116.049999 69.930001) (width 0.4) (layer B.Cu) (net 6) (status 10))
 (segment (start 116.049999 79.727999) (end 118.11 81.788) (width 0.4) (layer B.Cu) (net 6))
 (via (at 118.11 81.788) (size 0.5) (drill 0.3) (layers F.Cu B.Cu) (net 6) (status 30))
 (segment (start 133.610002 89.66) (end 133.32 89.66) (width 0.4) (layer F.Cu) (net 14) (status 30))
 (segment (start 134.870001 88.400001) (end 133.610002 89.66) (width 0.4) (layer F.Cu) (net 14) (status 20))
 (segment (start 134.870001 75.872001) (end 134.870001 88.400001) (width 0.4) (layer F.Cu) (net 14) (status 10))
 (segment (start 134.4168 75.4188) (end 134.870001 75.872001) (width 0.4) (layer F.Cu) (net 14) (status 30))
 (segment (start 127.7874 77.0926) (end 126.72 78.16) (width 0.5) (layer F.Cu) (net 11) (status 20))
 (segment (start 127.7874 75.3488) (end 127.7874 77.0926) (width 0.5) (layer F.Cu) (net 11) (status 10))
 (segment (start 125.5268 77.3532) (end 124.72 78.16) (width 0.5) (layer F.Cu) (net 10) (status 20))
 (segment (start 125.5268 75.368) (end 125.5268 77.3532) (width 0.5) (layer F.Cu) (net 10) (status 10))
 (segment (start 124.477599 74.318799) (end 125.5268 75.368) (width 0.5) (layer F.Cu) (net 10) (status 20))
 (segment (start 120.825201 74.318799) (end 124.477599 74.318799) (width 0.5) (layer F.Cu) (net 10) (status 10))
 (segment (start 120.396 74.748) (end 120.825201 74.318799) (width 0.5) (layer F.Cu) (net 10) (status 30))
 (segment (start 131.39 66.5) (end 131.318 66.428) (width 0.5) (layer B.Cu) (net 2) (status 30))
 (segment (start 133.4 66.5) (end 131.39 66.5) (width 0.5) (layer B.Cu) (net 2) (status 30))
 (segment (start 131.318 67.684) (end 132.08 68.446) (width 0.5) (layer B.Cu) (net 2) (status 20))
 (segment (start 131.318 66.428) (end 131.318 67.684) (width 0.5) (layer B.Cu) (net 2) (status 10))
 (segment (start 133.52 68.446) (end 133.67 68.296) (width 0.5) (layer B.Cu) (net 2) (status 30))
 (segment (start 132.08 68.446) (end 133.52 68.446) (width 0.5) (layer B.Cu) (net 2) (status 30))
 (segment (start 131.179999 69.346001) (end 132.08 68.446) (width 0.5) (layer B.Cu) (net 2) (status 20))
 (segment (start 131.179999 71.776001) (end 131.179999 69.346001) (width 0.5) (layer B.Cu) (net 2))
 (segment (start 133.422999 73.478999) (end 131.790001 71.846001) (width 0.5) (layer B.Cu) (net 2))
 (segment (start 131.790001 71.846001) (end 131.249999 71.846001) (width 0.5) (layer B.Cu) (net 2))
 (segment (start 133.422999 73.809999) (end 133.422999 73.478999) (width 0.5) (layer B.Cu) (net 2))
 (segment (start 131.249999 71.846001) (end 131.179999 71.776001) (width 0.5) (layer B.Cu) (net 2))
 (segment (start 134.223 74.61) (end 133.422999 73.809999) (width 0.5) (layer B.Cu) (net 2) (status 10))
 (segment (start 123 62) (end 129.5 62) (width 0.5) (layer F.Cu) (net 2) (status 30))
 (segment (start 131.318 66.058002) (end 131.318 66.428) (width 0.5) (layer B.Cu) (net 2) (status 30))
 (segment (start 129.5 64.240002) (end 131.318 66.058002) (width 0.5) (layer B.Cu) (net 2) (status 20))
 (segment (start 129.5 62) (end 129.5 64.240002) (width 0.5) (layer B.Cu) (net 2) (status 10))
 (segment (start 130.048 76.832) (end 128.72 78.16) (width 0.5) (layer F.Cu) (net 12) (status 20))
 (segment (start 130.048 75.3488) (end 130.048 76.832) (width 0.5) (layer F.Cu) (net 12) (status 10))
 (segment (start 129.90976 87.02044) (end 130.03276 87.14344) (width 0.5) (layer B.Cu) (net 16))
 (segment (start 127.13776 87.02044) (end 129.90976 87.02044) (width 0.5) (layer B.Cu) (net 16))
 (via (at 122.682 78.232) (size 0.8) (drill 0.4) (layers F.Cu B.Cu) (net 9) (status 30))
 (segment (start 135.57 72.182) (end 135.89 72.502) (width 0.5) (layer B.Cu) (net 9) (status 20))
 (segment (start 135.57 70.896) (end 135.57 72.182) (width 0.5) (layer B.Cu) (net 9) (status 10))
 (segment (start 122.682 78.232) (end 122.682 70.866) (width 0.25) (layer B.Cu) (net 9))
 (segment (start 122.682 70.866) (end 122.809 70.739) (width 0.25) (layer B.Cu) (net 9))
 (segment (start 122.809 70.739) (end 129.109 70.739) (width 0.25) (layer B.Cu) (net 9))
 (via (at 129.109 70.739) (size 0.5) (drill 0.3) (layers F.Cu B.Cu) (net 9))
 (segment (start 129.109 70.739) (end 135.459 70.739) (width 0.25) (layer F.Cu) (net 9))
 (via (at 135.459 70.739) (size 0.5) (drill 0.3) (layers F.Cu B.Cu) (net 9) (status 30))
 (segment (start 125.1718 71.247) (end 123.4 73.0188) (width 0.5) (layer F.Cu) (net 4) (status 30))
 (segment (start 125.349 71.247) (end 125.1718 71.247) (width 0.5) (layer F.Cu) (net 4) (status 30))
 (segment (start 123.4 75.48) (end 120.72 78.16) (width 0.5) (layer F.Cu) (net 8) (status 30))
 (segment (start 123.4 75.4188) (end 123.4 75.48) (width 0.5) (layer F.Cu) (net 8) (status 30))
 (via (at 132.207 61.595) (size 0.5) (drill 0.3) (layers F.Cu B.Cu) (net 18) (status 30))
 (via (at 134.239 61.722) (size 0.5) (drill 0.3) (layers F.Cu B.Cu) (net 17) (status 30))
 (segment (start 135.636 68.23) (end 135.57 68.296) (width 0.5) (layer B.Cu) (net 17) (status 30))
 (segment (start 135.636 66.478) (end 135.636 66.548) (width 0.5) (layer B.Cu) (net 17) (status 30))
 (segment (start 135.636 66.548) (end 135.636 68.23) (width 0.5) (layer B.Cu) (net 17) (status 30))
 (via (at 135.636 66.548) (size 0.5) (drill 0.3) (layers F.Cu B.Cu) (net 17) (status 30))
 (segment (start 135.636 66.548) (end 135.636 64.262) (width 0.5) (layer F.Cu) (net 17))
 (segment (start 134.239 62.865) (end 134.239 61.722) (width 0.5) (layer F.Cu) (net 17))
 (segment (start 135.636 64.262) (end 134.239 62.865) (width 0.5) (layer F.Cu) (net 17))
 (segment (start 123 66.5) (end 129.5 66.5) (width 0.5) (layer F.Cu) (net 17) (status 30))
 (segment (start 133.55401 63.54999) (end 134.239 62.865) (width 0.5) (layer F.Cu) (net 17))
 (segment (start 132.45001 63.54999) (end 133.55401 63.54999) (width 0.5) (layer F.Cu) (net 17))
 (segment (start 129.5 66.5) (end 132.45001 63.54999) (width 0.5) (layer F.Cu) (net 17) (status 10))
 (segment (start 129.65576 85.12044) (end 130.03276 84.74344) (width 0.5) (layer B.Cu) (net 1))
 (segment (start 127.13776 85.12044) (end 129.65576 85.12044) (width 0.5) (layer B.Cu) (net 1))
 (segment (start 132.223 74.090002) (end 135.26516 77.132162) (width 0.5) (layer B.Cu) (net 1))
 (segment (start 132.223 73.66) (end 132.223 74.090002) (width 0.5) (layer B.Cu) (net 1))
 (segment (start 135.26516 77.132162) (end 135.26516 81.80324) (width 0.5) (layer B.Cu) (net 1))
 (segment (start 132.32496 84.74344) (end 130.03276 84.74344) (width 0.5) (layer B.Cu) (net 1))
 (segment (start 135.26516 81.80324) (end 132.32496 84.74344) (width 0.5) (layer B.Cu) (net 1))
 (segment (start 134.62 72.313) (end 134.223 72.71) (width 0.5) (layer B.Cu) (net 3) (status 30))
 (segment (start 134.62 70.896) (end 134.62 72.313) (width 0.5) (layer B.Cu) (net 3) (status 30)))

